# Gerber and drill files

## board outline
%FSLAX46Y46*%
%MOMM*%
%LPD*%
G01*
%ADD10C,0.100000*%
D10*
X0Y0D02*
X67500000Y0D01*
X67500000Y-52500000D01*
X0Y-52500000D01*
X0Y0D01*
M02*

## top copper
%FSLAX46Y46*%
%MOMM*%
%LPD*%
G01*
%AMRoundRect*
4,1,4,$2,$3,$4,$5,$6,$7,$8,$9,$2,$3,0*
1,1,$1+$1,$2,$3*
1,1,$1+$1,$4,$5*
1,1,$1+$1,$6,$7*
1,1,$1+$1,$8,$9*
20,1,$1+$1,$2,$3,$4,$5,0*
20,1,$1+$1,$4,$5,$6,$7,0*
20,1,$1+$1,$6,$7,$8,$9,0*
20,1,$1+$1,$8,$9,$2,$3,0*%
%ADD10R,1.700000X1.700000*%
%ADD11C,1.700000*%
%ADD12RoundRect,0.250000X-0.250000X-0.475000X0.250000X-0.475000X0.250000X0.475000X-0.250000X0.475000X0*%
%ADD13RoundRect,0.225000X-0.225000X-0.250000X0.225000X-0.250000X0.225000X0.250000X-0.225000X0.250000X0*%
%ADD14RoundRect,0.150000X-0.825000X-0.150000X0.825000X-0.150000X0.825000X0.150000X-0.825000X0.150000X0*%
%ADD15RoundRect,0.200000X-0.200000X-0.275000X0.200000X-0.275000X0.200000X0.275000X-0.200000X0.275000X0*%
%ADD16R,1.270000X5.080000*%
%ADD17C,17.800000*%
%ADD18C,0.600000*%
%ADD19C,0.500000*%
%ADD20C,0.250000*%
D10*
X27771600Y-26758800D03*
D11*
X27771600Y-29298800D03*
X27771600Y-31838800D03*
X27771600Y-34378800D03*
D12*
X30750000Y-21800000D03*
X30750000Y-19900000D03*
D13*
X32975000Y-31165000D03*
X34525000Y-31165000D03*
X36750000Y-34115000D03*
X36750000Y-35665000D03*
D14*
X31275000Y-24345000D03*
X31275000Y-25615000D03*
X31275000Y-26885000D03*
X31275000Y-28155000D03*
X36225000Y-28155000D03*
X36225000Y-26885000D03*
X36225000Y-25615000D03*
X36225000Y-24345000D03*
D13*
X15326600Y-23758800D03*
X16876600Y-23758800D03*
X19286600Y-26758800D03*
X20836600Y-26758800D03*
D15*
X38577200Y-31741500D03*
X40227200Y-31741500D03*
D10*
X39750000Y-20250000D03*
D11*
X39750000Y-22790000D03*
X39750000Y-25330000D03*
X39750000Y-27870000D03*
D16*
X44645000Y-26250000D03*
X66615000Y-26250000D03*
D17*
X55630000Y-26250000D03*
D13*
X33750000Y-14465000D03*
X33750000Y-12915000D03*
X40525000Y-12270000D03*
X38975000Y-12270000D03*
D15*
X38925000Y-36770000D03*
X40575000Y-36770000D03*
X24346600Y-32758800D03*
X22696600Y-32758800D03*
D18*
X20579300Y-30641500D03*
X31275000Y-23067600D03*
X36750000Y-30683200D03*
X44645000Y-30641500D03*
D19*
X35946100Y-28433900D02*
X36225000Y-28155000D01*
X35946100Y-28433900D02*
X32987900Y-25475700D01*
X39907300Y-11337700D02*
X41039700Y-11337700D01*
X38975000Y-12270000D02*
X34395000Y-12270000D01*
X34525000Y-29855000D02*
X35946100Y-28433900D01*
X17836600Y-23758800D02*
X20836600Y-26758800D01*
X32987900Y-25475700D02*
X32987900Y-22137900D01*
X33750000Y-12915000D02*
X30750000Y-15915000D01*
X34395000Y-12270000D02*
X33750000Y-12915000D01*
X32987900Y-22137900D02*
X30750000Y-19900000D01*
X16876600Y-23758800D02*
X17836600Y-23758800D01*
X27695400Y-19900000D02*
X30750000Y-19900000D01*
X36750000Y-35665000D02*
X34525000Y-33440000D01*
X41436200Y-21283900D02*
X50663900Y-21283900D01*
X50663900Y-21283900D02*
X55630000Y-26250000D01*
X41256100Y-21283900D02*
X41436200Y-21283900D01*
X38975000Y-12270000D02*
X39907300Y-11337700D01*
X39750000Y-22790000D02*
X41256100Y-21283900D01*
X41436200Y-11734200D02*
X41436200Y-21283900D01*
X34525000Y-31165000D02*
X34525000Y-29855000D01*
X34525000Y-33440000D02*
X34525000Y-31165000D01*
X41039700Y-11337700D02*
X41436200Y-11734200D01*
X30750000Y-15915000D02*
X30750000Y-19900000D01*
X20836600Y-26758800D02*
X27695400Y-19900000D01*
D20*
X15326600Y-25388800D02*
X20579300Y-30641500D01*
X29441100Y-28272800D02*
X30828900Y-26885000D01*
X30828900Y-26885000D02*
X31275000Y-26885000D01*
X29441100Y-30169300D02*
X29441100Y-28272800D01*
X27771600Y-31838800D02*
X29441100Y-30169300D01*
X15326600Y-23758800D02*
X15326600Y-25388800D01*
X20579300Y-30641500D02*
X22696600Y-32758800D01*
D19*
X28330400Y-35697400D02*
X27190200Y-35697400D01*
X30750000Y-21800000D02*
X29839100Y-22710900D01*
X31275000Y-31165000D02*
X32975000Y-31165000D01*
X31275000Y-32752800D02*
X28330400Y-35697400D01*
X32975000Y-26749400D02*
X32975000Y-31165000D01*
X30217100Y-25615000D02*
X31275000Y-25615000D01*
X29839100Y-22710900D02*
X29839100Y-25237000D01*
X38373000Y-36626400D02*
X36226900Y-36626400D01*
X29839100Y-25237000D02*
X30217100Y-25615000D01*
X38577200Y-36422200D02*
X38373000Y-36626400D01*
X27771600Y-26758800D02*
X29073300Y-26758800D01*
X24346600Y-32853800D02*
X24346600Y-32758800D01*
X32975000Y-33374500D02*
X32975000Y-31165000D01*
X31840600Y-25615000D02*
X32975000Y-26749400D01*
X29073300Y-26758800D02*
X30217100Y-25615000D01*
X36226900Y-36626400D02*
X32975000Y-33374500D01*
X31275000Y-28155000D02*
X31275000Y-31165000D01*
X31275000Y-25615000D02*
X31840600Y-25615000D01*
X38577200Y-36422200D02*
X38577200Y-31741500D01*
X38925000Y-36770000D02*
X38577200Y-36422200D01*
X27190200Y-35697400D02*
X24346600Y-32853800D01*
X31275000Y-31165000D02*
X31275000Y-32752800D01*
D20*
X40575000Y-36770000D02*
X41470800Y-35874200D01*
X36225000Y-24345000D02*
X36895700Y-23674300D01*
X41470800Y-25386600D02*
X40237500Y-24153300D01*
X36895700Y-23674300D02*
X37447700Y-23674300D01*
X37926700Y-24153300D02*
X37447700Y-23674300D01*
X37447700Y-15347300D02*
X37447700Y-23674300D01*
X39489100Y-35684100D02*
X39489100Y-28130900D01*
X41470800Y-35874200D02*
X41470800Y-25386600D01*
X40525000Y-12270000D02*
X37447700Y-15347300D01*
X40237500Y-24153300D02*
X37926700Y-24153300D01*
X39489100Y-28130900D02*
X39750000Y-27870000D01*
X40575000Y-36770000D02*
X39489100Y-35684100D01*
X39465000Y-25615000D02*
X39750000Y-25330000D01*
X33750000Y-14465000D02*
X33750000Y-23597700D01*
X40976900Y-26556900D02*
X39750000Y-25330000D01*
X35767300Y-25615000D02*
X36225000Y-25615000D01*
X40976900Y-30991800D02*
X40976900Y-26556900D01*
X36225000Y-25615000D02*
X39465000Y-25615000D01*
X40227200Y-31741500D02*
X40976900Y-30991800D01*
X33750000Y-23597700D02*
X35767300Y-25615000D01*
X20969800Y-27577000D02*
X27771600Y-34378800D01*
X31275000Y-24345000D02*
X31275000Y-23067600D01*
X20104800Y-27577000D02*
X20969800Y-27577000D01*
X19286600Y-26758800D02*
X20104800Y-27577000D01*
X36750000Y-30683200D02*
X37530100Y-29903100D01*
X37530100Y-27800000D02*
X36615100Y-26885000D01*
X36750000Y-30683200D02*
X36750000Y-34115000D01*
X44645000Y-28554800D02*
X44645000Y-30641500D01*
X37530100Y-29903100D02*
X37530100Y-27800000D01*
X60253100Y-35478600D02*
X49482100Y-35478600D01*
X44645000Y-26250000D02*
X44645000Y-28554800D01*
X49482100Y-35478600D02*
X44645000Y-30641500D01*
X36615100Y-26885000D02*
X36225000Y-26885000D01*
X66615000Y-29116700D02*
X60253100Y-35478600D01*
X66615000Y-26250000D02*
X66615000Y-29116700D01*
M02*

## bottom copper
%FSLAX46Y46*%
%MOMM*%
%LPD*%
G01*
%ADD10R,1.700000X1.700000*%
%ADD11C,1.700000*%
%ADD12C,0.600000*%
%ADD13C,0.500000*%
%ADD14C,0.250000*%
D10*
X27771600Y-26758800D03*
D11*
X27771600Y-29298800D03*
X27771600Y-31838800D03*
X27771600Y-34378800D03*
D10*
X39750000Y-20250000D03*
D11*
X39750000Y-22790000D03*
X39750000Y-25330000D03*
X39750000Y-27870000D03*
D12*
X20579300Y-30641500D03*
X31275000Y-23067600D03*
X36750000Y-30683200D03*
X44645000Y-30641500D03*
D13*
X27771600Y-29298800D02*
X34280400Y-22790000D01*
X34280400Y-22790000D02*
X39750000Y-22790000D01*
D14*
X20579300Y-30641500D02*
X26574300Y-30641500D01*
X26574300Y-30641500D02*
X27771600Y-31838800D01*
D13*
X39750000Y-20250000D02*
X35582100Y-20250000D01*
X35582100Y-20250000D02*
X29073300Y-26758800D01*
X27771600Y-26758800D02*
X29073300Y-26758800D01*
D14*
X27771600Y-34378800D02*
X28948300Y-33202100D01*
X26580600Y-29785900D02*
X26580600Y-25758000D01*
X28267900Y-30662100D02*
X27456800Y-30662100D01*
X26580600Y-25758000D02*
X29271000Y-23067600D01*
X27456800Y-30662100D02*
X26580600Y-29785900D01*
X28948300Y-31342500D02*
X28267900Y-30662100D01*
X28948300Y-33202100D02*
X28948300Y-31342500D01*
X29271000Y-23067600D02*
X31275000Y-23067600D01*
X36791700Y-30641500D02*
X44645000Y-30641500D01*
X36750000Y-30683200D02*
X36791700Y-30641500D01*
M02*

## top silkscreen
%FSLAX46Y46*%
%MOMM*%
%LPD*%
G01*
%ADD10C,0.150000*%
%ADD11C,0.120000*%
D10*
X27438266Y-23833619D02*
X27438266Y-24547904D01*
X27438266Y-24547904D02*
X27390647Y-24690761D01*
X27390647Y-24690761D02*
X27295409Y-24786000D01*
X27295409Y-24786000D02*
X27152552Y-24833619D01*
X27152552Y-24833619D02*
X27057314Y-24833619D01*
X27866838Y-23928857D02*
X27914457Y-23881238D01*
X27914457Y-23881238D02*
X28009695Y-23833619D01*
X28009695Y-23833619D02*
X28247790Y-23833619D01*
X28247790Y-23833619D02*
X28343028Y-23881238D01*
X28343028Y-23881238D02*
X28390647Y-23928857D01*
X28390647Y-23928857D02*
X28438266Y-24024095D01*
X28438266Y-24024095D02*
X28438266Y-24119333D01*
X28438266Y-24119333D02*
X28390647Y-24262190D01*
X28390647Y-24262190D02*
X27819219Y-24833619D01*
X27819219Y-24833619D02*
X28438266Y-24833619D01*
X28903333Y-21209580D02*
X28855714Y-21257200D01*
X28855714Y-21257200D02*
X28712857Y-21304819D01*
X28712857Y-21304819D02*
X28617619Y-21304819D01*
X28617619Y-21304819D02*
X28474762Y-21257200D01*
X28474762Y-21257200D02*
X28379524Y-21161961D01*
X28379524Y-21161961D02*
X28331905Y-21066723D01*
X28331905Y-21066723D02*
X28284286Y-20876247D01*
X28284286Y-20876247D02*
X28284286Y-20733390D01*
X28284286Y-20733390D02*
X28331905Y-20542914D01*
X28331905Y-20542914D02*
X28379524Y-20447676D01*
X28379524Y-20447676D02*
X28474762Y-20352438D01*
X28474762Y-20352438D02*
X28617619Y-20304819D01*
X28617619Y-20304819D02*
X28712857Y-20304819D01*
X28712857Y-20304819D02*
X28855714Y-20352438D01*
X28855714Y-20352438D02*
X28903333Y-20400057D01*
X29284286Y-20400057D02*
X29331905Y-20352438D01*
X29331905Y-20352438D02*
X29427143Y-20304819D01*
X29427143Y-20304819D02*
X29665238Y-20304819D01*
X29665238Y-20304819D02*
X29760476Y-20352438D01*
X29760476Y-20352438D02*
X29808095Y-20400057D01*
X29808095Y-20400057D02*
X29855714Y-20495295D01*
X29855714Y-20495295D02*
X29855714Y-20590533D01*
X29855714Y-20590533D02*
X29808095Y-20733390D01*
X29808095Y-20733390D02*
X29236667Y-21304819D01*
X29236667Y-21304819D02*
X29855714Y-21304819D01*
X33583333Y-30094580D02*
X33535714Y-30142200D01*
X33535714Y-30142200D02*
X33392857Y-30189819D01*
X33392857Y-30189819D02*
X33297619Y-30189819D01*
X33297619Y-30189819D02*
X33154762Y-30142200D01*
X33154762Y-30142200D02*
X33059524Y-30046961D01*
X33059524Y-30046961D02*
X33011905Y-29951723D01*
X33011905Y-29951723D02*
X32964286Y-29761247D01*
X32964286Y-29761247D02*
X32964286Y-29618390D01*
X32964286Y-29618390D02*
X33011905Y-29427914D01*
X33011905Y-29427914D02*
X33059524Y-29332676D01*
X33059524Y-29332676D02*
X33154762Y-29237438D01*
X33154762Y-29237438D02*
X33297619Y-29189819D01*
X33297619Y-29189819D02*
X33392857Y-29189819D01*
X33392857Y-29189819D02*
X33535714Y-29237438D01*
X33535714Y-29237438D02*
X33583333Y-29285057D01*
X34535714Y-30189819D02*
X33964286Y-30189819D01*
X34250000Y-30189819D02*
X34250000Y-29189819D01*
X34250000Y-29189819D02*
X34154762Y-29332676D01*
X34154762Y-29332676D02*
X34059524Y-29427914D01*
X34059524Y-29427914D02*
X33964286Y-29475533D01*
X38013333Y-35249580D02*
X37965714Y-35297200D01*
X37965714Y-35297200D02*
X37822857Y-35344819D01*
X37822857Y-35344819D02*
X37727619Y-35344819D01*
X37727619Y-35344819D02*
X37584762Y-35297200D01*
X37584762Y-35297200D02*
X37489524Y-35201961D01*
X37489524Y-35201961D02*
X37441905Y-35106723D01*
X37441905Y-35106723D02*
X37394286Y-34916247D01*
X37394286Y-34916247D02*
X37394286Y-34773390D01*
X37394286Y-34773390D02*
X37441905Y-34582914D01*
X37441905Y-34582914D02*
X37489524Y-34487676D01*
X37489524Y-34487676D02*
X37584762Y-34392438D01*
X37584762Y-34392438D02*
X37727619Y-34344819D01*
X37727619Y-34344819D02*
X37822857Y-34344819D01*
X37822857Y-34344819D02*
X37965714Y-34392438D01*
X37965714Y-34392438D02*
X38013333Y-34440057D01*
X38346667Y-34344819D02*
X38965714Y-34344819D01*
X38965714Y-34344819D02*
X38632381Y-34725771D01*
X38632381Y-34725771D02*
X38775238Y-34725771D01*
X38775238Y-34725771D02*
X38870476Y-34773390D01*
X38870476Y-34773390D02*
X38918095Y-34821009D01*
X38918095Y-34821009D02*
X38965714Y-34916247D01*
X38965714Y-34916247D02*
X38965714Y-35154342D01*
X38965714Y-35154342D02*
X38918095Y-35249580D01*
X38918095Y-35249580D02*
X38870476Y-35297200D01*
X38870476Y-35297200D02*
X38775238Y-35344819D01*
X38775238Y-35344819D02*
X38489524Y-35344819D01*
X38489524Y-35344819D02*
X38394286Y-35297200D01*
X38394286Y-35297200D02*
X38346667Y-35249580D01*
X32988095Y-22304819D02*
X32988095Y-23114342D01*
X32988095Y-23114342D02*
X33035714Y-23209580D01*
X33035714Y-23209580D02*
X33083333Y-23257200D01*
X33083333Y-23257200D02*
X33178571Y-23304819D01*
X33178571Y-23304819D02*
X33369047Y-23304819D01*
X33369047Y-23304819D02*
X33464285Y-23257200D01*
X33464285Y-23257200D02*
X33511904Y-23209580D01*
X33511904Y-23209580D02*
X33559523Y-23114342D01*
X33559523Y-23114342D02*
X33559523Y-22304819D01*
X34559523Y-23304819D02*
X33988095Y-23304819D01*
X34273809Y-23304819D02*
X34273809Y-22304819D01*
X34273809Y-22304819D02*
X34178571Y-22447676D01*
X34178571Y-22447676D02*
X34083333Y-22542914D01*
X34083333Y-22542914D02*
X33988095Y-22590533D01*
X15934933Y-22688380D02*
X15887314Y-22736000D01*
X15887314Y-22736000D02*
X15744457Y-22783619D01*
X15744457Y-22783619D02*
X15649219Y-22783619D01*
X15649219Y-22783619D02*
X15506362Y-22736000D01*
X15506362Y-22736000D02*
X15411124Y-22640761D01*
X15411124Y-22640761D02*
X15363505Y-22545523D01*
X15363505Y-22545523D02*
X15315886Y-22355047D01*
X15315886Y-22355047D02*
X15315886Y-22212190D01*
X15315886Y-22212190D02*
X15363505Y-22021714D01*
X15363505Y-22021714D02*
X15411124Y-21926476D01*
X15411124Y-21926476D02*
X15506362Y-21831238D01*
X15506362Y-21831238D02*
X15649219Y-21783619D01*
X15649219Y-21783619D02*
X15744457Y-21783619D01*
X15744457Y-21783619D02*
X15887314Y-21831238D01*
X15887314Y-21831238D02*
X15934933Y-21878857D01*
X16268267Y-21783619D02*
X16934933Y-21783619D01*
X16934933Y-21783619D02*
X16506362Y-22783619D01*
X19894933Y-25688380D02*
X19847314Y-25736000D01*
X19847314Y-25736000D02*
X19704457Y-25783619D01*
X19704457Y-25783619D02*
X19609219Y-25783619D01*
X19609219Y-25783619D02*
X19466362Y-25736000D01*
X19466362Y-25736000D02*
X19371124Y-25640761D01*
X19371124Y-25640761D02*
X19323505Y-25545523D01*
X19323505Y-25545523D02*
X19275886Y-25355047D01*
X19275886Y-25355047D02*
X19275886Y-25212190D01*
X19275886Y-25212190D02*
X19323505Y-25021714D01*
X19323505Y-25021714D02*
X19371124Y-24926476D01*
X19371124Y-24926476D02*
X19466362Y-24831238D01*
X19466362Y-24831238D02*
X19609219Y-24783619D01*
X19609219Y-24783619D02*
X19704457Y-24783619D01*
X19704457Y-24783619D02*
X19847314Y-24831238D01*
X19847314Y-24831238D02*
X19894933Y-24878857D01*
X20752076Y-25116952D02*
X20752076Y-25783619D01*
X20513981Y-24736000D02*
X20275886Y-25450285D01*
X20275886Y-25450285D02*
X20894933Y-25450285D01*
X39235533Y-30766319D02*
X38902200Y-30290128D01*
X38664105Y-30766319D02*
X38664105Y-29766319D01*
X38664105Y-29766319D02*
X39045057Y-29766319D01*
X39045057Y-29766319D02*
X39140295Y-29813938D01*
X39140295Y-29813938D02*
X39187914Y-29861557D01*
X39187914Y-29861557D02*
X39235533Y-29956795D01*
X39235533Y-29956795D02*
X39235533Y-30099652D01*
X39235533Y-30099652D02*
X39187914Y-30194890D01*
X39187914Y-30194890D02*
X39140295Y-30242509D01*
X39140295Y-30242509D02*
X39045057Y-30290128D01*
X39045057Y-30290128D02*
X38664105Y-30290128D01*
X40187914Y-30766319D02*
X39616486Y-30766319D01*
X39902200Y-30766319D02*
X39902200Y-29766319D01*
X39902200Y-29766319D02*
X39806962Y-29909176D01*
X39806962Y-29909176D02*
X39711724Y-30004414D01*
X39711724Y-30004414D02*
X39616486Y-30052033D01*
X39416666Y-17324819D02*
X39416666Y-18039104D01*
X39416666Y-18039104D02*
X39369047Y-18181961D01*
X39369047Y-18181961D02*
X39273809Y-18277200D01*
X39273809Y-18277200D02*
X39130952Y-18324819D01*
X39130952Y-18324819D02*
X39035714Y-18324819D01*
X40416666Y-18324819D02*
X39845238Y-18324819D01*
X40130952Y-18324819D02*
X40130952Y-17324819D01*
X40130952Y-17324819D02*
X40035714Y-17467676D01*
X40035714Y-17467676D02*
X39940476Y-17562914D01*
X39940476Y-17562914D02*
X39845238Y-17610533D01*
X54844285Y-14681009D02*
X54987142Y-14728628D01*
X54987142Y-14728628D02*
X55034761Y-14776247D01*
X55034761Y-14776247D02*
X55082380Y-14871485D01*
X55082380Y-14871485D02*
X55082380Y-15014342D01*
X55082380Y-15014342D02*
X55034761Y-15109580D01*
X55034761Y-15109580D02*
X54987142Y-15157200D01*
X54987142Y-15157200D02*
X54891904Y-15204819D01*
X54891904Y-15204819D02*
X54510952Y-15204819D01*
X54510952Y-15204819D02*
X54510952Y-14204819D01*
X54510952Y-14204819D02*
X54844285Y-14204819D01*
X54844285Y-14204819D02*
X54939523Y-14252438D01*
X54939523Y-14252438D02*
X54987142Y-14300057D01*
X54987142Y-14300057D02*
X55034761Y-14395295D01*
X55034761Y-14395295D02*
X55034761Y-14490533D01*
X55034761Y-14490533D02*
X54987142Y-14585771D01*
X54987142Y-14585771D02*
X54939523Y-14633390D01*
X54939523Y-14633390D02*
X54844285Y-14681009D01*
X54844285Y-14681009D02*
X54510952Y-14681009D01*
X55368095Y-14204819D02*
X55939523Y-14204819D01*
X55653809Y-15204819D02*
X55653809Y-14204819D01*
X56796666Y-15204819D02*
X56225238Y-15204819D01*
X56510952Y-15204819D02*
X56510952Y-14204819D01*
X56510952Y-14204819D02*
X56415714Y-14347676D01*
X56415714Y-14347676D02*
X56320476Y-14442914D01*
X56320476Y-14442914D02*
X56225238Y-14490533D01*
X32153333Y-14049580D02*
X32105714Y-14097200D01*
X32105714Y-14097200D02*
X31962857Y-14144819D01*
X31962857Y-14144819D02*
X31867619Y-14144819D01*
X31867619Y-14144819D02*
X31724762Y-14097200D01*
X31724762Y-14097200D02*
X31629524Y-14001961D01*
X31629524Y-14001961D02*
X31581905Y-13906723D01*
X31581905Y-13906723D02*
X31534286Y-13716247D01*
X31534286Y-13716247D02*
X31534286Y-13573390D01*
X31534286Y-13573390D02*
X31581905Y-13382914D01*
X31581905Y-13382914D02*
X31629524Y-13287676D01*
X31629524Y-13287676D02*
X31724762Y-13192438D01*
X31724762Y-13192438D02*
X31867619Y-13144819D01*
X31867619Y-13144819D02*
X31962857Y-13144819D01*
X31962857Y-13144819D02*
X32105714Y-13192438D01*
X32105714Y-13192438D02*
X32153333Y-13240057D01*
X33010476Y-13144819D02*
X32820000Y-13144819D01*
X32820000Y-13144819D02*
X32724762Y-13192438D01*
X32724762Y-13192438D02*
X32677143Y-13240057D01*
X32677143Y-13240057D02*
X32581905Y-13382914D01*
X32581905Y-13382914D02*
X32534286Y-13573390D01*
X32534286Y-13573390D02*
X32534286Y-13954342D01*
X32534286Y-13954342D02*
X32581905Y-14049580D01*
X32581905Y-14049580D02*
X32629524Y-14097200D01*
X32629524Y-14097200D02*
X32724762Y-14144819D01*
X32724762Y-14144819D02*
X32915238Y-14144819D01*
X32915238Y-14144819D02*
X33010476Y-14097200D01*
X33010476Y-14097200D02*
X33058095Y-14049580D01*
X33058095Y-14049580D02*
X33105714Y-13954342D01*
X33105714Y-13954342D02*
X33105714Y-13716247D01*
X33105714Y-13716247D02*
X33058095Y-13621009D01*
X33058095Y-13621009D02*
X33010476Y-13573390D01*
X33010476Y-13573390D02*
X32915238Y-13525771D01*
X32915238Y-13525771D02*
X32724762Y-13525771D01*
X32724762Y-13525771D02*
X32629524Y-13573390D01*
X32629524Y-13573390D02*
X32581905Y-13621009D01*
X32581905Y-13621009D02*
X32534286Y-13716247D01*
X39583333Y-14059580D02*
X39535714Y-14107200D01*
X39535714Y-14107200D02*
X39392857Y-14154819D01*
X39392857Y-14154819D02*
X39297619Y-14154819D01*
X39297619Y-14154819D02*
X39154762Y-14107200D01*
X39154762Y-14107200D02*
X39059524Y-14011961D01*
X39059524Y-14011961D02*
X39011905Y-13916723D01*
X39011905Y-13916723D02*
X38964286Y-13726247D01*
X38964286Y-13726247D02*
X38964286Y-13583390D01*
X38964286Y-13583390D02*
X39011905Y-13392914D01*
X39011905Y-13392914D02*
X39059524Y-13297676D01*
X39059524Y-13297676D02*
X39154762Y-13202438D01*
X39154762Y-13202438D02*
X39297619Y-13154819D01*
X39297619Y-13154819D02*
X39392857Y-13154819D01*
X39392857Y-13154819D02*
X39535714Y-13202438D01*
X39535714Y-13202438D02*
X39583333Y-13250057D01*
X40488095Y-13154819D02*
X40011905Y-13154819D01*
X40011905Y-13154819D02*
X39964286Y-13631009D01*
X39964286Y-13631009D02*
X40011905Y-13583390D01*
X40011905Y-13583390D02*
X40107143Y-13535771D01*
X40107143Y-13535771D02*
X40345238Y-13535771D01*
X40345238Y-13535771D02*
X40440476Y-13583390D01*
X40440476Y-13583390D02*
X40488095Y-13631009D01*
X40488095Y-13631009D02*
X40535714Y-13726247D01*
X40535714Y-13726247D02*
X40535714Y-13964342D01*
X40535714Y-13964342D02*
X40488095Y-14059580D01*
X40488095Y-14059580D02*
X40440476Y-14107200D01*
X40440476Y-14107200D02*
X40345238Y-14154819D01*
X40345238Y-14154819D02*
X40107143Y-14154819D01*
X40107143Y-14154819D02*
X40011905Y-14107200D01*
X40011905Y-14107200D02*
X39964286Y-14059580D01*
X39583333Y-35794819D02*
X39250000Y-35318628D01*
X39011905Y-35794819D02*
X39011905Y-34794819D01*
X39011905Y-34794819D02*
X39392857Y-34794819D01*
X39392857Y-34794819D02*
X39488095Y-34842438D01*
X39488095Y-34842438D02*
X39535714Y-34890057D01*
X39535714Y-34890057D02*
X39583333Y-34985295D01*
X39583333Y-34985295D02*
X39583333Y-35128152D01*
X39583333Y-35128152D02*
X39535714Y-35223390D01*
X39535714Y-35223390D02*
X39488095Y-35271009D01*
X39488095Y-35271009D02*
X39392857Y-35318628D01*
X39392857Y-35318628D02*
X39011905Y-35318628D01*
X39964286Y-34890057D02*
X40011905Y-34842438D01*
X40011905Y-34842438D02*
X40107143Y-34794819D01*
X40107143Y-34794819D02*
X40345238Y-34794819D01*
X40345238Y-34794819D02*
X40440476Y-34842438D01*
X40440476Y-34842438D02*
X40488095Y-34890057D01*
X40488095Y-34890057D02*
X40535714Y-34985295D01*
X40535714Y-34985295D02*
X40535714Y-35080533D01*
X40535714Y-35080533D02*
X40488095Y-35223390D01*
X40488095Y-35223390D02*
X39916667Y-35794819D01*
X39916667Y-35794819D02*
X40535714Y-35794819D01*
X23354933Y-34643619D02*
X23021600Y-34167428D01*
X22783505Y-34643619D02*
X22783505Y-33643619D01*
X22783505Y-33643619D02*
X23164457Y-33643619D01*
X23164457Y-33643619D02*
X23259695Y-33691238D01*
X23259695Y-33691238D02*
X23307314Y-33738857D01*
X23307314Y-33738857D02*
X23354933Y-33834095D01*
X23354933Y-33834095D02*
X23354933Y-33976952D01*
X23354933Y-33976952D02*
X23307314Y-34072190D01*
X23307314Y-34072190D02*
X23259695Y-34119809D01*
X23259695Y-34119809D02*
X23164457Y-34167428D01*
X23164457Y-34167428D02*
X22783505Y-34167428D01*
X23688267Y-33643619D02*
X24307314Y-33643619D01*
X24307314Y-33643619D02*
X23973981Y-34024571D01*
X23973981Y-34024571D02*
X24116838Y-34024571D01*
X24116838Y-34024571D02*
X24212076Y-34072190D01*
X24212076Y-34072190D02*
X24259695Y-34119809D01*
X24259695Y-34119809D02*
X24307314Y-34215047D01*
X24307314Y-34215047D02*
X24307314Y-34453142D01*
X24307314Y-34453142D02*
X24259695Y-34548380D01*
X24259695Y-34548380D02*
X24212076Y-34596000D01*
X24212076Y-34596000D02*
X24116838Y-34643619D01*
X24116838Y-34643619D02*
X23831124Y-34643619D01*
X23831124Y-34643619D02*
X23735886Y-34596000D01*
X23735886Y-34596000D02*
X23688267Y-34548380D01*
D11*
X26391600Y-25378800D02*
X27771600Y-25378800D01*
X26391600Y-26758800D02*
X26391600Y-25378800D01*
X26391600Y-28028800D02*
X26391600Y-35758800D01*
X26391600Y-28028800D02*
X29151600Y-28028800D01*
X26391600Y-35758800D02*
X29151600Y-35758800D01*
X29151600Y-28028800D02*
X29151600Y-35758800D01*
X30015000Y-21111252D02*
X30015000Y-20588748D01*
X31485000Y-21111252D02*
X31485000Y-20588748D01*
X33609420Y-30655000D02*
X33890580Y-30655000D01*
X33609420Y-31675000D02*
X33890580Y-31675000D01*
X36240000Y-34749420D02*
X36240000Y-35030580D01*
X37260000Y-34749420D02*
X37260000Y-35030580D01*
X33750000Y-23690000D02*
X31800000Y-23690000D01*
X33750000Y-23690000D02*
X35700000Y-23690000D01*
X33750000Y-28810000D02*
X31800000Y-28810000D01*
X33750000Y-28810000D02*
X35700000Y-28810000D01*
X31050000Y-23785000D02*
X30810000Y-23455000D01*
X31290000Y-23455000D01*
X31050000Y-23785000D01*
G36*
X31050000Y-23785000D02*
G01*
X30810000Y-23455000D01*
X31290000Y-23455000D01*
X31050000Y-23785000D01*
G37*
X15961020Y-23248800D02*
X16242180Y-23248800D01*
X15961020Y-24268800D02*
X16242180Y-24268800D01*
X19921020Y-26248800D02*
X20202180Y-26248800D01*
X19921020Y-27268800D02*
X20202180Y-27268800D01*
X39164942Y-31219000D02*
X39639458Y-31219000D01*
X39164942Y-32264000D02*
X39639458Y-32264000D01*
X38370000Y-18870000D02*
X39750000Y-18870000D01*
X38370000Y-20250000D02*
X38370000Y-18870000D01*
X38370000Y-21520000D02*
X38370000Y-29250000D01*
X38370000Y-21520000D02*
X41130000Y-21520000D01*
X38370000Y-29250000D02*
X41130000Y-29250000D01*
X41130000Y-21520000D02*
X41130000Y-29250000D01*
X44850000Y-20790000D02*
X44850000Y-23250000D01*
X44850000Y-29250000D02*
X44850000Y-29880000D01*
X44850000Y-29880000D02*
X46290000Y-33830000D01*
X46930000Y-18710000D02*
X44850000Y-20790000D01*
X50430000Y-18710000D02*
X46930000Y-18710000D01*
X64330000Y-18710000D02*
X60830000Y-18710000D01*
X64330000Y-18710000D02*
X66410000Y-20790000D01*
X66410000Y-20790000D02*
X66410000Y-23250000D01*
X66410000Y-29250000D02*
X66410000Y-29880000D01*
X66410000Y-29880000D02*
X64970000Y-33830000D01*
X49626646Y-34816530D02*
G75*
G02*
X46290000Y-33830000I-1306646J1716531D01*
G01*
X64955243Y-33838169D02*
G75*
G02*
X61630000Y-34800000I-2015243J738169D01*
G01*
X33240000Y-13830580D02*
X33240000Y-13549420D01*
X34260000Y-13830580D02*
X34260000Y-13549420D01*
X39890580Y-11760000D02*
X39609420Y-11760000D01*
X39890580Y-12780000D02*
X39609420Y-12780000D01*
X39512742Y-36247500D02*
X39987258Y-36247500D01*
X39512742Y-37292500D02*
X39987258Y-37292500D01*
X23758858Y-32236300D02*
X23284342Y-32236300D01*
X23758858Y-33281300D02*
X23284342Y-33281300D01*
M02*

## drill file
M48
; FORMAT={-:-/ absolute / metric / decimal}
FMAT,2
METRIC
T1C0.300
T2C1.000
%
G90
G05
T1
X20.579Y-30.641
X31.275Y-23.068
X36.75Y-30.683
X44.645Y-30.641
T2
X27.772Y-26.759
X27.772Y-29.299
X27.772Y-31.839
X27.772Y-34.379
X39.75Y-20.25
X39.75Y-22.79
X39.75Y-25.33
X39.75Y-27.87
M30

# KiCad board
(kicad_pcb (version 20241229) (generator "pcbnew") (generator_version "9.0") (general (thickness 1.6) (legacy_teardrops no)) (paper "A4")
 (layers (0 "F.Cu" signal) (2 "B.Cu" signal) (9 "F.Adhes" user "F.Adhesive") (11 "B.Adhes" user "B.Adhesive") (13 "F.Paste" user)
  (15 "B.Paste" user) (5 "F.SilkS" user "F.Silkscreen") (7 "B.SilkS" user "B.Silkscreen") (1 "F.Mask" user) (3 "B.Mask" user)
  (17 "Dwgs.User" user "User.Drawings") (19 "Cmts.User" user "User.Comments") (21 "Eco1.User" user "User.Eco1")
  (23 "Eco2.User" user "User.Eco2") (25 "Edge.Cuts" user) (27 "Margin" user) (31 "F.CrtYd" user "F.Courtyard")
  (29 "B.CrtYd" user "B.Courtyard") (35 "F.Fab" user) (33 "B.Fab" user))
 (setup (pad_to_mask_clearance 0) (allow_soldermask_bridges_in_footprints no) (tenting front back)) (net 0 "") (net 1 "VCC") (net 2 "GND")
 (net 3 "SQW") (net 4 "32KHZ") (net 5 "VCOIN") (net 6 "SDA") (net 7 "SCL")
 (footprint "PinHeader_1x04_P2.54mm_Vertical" (layer "F.Cu") (at 27.7716 26.7588)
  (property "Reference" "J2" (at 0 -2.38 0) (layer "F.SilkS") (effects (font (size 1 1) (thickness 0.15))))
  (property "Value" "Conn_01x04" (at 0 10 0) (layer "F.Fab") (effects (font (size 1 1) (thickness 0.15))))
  (fp_line (start -1.38 -1.38) (end 0 -1.38) (stroke (width 0.12) (type solid)) (layer "F.SilkS"))
  (fp_line (start -1.38 0) (end -1.38 -1.38) (stroke (width 0.12) (type solid)) (layer "F.SilkS"))
  (fp_line (start -1.38 1.27) (end -1.38 9) (stroke (width 0.12) (type solid)) (layer "F.SilkS"))
  (fp_line (start -1.38 1.27) (end 1.38 1.27) (stroke (width 0.12) (type solid)) (layer "F.SilkS"))
  (fp_line (start -1.38 9) (end 1.38 9) (stroke (width 0.12) (type solid)) (layer "F.SilkS"))
  (fp_line (start 1.38 1.27) (end 1.38 9) (stroke (width 0.12) (type solid)) (layer "F.SilkS"))
  (pad "1" thru_hole rect (at 0 0) (size 1.7 1.7) (drill 1) (layers "*.Cu" "*.Mask") (remove_unused_layers no) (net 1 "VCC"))
  (pad "2" thru_hole circle (at 0 2.54) (size 1.7 1.7) (drill 1) (layers "*.Cu" "*.Mask") (remove_unused_layers no) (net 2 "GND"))
  (pad "3" thru_hole circle (at 0 5.08) (size 1.7 1.7) (drill 1) (layers "*.Cu" "*.Mask") (remove_unused_layers no) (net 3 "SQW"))
  (pad "4" thru_hole circle (at 0 7.62) (size 1.7 1.7) (drill 1) (layers "*.Cu" "*.Mask") (remove_unused_layers no) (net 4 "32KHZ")))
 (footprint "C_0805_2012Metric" (layer "F.Cu") (at 30.75 20.85 90)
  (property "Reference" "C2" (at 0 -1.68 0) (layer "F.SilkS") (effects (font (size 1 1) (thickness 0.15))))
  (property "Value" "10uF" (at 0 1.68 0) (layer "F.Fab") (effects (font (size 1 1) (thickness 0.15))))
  (fp_line (start -0.261252 -0.735) (end 0.261252 -0.735) (stroke (width 0.12) (type solid)) (layer "F.SilkS"))
  (fp_line (start -0.261252 0.735) (end 0.261252 0.735) (stroke (width 0.12) (type solid)) (layer "F.SilkS"))
  (pad "1" smd roundrect (at -0.95 0) (size 1 1.45) (layers "F.Cu" "F.Mask" "F.Paste") (roundrect_rratio 0.25) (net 1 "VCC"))
  (pad "2" smd roundrect (at 0.95 0) (size 1 1.45) (layers "F.Cu" "F.Mask" "F.Paste") (roundrect_rratio 0.25) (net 2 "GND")))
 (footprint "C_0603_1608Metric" (layer "F.Cu") (at 33.75 31.165)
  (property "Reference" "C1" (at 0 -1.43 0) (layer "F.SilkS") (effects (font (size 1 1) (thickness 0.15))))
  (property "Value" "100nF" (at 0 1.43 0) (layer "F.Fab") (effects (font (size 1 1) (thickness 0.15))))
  (fp_line (start -0.14058 -0.51) (end 0.14058 -0.51) (stroke (width 0.12) (type solid)) (layer "F.SilkS"))
  (fp_line (start -0.14058 0.51) (end 0.14058 0.51) (stroke (width 0.12) (type solid)) (layer "F.SilkS"))
  (pad "1" smd roundrect (at -0.775 0) (size 0.9 0.95) (layers "F.Cu" "F.Mask" "F.Paste") (roundrect_rratio 0.25) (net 1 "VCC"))
  (pad "2" smd roundrect (at 0.775 0) (size 0.9 0.95) (layers "F.Cu" "F.Mask" "F.Paste") (roundrect_rratio 0.25) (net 2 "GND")))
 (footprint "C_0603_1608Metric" (layer "F.Cu") (at 36.75 34.89 -90)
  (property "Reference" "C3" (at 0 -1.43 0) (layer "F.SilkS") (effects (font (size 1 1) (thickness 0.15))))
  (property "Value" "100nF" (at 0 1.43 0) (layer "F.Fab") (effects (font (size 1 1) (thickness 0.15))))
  (fp_line (start -0.14058 0.51) (end 0.14058 0.51) (stroke (width 0.12) (type solid)) (layer "F.SilkS"))
  (fp_line (start -0.14058 -0.51) (end 0.14058 -0.51) (stroke (width 0.12) (type solid)) (layer "F.SilkS"))
  (pad "1" smd roundrect (at -0.775 0) (size 0.9 0.95) (layers "F.Cu" "F.Mask" "F.Paste") (roundrect_rratio 0.25) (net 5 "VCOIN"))
  (pad "2" smd roundrect (at 0.775 0) (size 0.9 0.95) (layers "F.Cu" "F.Mask" "F.Paste") (roundrect_rratio 0.25) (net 2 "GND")))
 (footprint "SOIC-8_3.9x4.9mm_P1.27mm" (layer "F.Cu") (at 33.75 26.25)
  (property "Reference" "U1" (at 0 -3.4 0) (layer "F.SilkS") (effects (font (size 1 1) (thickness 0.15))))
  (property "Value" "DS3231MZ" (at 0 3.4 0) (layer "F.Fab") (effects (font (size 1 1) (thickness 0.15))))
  (fp_line (start 0 -2.56) (end -1.95 -2.56) (stroke (width 0.12) (type solid)) (layer "F.SilkS"))
  (fp_line (start 0 -2.56) (end 1.95 -2.56) (stroke (width 0.12) (type solid)) (layer "F.SilkS"))
  (fp_line (start 0 2.56) (end -1.95 2.56) (stroke (width 0.12) (type solid)) (layer "F.SilkS"))
  (fp_line (start 0 2.56) (end 1.95 2.56) (stroke (width 0.12) (type solid)) (layer "F.SilkS"))
  (fp_poly (pts (xy -2.7 -2.465) (xy -2.94 -2.795) (xy -2.46 -2.795)) (stroke (width 0.12) (type solid)) (fill yes) (layer "F.SilkS"))
  (pad "1" smd roundrect (at -2.475 -1.905) (size 1.95 0.6) (layers "F.Cu" "F.Mask" "F.Paste") (roundrect_rratio 0.25) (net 4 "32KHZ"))
  (pad "2" smd roundrect (at -2.475 -0.635) (size 1.95 0.6) (layers "F.Cu" "F.Mask" "F.Paste") (roundrect_rratio 0.25) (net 1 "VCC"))
  (pad "3" smd roundrect (at -2.475 0.635) (size 1.95 0.6) (layers "F.Cu" "F.Mask" "F.Paste") (roundrect_rratio 0.25) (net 3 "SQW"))
  (pad "4" smd roundrect (at -2.475 1.905) (size 1.95 0.6) (layers "F.Cu" "F.Mask" "F.Paste") (roundrect_rratio 0.25) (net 1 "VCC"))
  (pad "5" smd roundrect (at 2.475 1.905) (size 1.95 0.6) (layers "F.Cu" "F.Mask" "F.Paste") (roundrect_rratio 0.25) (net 2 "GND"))
  (pad "6" smd roundrect (at 2.475 0.635) (size 1.95 0.6) (layers "F.Cu" "F.Mask" "F.Paste") (roundrect_rratio 0.25) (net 5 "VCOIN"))
  (pad "7" smd roundrect (at 2.475 -0.635) (size 1.95 0.6) (layers "F.Cu" "F.Mask" "F.Paste") (roundrect_rratio 0.25) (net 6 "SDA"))
  (pad "8" smd roundrect (at 2.475 -1.905) (size 1.95 0.6) (layers "F.Cu" "F.Mask" "F.Paste") (roundrect_rratio 0.25) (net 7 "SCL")))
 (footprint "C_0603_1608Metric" (layer "F.Cu") (at 16.1016 23.7588)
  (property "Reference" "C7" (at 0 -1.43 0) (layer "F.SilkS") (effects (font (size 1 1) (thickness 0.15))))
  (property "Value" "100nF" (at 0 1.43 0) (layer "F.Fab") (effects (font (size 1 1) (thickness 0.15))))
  (fp_line (start -0.14058 -0.51) (end 0.14058 -0.51) (stroke (width 0.12) (type solid)) (layer "F.SilkS"))
  (fp_line (start -0.14058 0.51) (end 0.14058 0.51) (stroke (width 0.12) (type solid)) (layer "F.SilkS"))
  (pad "1" smd roundrect (at -0.775 0) (size 0.9 0.95) (layers "F.Cu" "F.Mask" "F.Paste") (roundrect_rratio 0.25) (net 3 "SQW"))
  (pad "2" smd roundrect (at 0.775 0) (size 0.9 0.95) (layers "F.Cu" "F.Mask" "F.Paste") (roundrect_rratio 0.25) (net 2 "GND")))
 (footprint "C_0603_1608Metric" (layer "F.Cu") (at 20.0616 26.7588)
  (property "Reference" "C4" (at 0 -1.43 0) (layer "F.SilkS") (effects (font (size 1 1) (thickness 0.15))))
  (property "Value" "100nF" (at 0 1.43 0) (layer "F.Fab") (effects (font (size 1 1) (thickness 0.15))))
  (fp_line (start -0.14058 -0.51) (end 0.14058 -0.51) (stroke (width 0.12) (type solid)) (layer "F.SilkS"))
  (fp_line (start -0.14058 0.51) (end 0.14058 0.51) (stroke (width 0.12) (type solid)) (layer "F.SilkS"))
  (pad "1" smd roundrect (at -0.775 0) (size 0.9 0.95) (layers "F.Cu" "F.Mask" "F.Paste") (roundrect_rratio 0.25) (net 4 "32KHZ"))
  (pad "2" smd roundrect (at 0.775 0) (size 0.9 0.95) (layers "F.Cu" "F.Mask" "F.Paste") (roundrect_rratio 0.25) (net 2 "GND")))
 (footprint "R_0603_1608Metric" (layer "F.Cu") (at 39.4022 31.7415)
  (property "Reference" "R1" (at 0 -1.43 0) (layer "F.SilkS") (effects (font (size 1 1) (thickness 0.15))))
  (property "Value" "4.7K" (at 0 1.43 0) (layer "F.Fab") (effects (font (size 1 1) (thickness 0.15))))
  (fp_line (start -0.237258 -0.5225) (end 0.237258 -0.5225) (stroke (width 0.12) (type solid)) (layer "F.SilkS"))
  (fp_line (start -0.237258 0.5225) (end 0.237258 0.5225) (stroke (width 0.12) (type solid)) (layer "F.SilkS"))
  (pad "1" smd roundrect (at -0.825 0) (size 0.8 0.95) (layers "F.Cu" "F.Mask" "F.Paste") (roundrect_rratio 0.25) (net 1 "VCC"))
  (pad "2" smd roundrect (at 0.825 0) (size 0.8 0.95) (layers "F.Cu" "F.Mask" "F.Paste") (roundrect_rratio 0.25) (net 6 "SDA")))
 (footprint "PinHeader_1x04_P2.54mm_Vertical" (layer "F.Cu") (at 39.75 20.25)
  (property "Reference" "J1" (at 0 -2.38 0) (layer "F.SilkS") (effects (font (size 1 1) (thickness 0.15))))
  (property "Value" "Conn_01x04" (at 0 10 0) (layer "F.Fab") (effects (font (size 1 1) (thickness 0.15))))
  (fp_line (start -1.38 -1.38) (end 0 -1.38) (stroke (width 0.12) (type solid)) (layer "F.SilkS"))
  (fp_line (start -1.38 0) (end -1.38 -1.38) (stroke (width 0.12) (type solid)) (layer "F.SilkS"))
  (fp_line (start -1.38 1.27) (end -1.38 9) (stroke (width 0.12) (type solid)) (layer "F.SilkS"))
  (fp_line (start -1.38 1.27) (end 1.38 1.27) (stroke (width 0.12) (type solid)) (layer "F.SilkS"))
  (fp_line (start -1.38 9) (end 1.38 9) (stroke (width 0.12) (type solid)) (layer "F.SilkS"))
  (fp_line (start 1.38 1.27) (end 1.38 9) (stroke (width 0.12) (type solid)) (layer "F.SilkS"))
  (pad "1" thru_hole rect (at 0 0) (size 1.7 1.7) (drill 1) (layers "*.Cu" "*.Mask") (remove_unused_layers no) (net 1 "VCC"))
  (pad "2" thru_hole circle (at 0 2.54) (size 1.7 1.7) (drill 1) (layers "*.Cu" "*.Mask") (remove_unused_layers no) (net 2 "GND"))
  (pad "3" thru_hole circle (at 0 5.08) (size 1.7 1.7) (drill 1) (layers "*.Cu" "*.Mask") (remove_unused_layers no) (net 6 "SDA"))
  (pad "4" thru_hole circle (at 0 7.62) (size 1.7 1.7) (drill 1) (layers "*.Cu" "*.Mask") (remove_unused_layers no) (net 7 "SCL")))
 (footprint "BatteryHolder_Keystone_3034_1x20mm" (layer "F.Cu") (at 55.63 26.25)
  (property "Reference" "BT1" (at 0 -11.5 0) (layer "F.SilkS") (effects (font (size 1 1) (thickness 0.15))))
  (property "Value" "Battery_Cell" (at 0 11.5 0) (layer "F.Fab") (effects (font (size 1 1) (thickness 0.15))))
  (fp_line (start -10.78 -5.46) (end -10.78 -3) (stroke (width 0.12) (type solid)) (layer "F.SilkS"))
  (fp_line (start -10.78 3) (end -10.78 3.63) (stroke (width 0.12) (type solid)) (layer "F.SilkS"))
  (fp_line (start -10.78 3.63) (end -9.34 7.58) (stroke (width 0.12) (type solid)) (layer "F.SilkS"))
  (fp_line (start -8.7 -7.54) (end -10.78 -5.46) (stroke (width 0.12) (type solid)) (layer "F.SilkS"))
  (fp_line (start -5.2 -7.54) (end -8.7 -7.54) (stroke (width 0.12) (type solid)) (layer "F.SilkS"))
  (fp_line (start 8.7 -7.54) (end 5.2 -7.54) (stroke (width 0.12) (type solid)) (layer "F.SilkS"))
  (fp_line (start 8.7 -7.54) (end 10.78 -5.46) (stroke (width 0.12) (type solid)) (layer "F.SilkS"))
  (fp_line (start 10.78 -5.46) (end 10.78 -3) (stroke (width 0.12) (type solid)) (layer "F.SilkS"))
  (fp_line (start 10.78 3) (end 10.78 3.63) (stroke (width 0.12) (type solid)) (layer "F.SilkS"))
  (fp_line (start 10.78 3.63) (end 9.34 7.58) (stroke (width 0.12) (type solid)) (layer "F.SilkS"))
  (fp_arc (start -6.003354 8.56653) (mid -7.921654 8.918738) (end -9.34 7.58) (stroke (width 0.12) (type solid)) (layer "F.SilkS"))
  (fp_arc (start 9.325243 7.588169) (mid 7.90634 8.911668) (end 6 8.55) (stroke (width 0.12) (type solid)) (layer "F.SilkS"))
  (pad "1" smd rect (at -10.985 0) (size 1.27 5.08) (layers "F.Cu" "F.Mask" "F.Paste") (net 5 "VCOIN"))
  (pad "1" smd rect (at 10.985 0) (size 1.27 5.08) (layers "F.Cu" "F.Mask" "F.Paste") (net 5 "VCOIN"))
  (pad "2" smd circle (at 0 0) (size 17.8 17.8) (layers "F.Cu" "F.Mask") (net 2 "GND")))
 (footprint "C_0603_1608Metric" (layer "F.Cu") (at 33.75 13.69 90)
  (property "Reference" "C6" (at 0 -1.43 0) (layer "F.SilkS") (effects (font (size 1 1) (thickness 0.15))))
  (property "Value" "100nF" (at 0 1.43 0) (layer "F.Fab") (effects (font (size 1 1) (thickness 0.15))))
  (fp_line (start -0.14058 -0.51) (end 0.14058 -0.51) (stroke (width 0.12) (type solid)) (layer "F.SilkS"))
  (fp_line (start -0.14058 0.51) (end 0.14058 0.51) (stroke (width 0.12) (type solid)) (layer "F.SilkS"))
  (pad "1" smd roundrect (at -0.775 0) (size 0.9 0.95) (layers "F.Cu" "F.Mask" "F.Paste") (roundrect_rratio 0.25) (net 6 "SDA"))
  (pad "2" smd roundrect (at 0.775 0) (size 0.9 0.95) (layers "F.Cu" "F.Mask" "F.Paste") (roundrect_rratio 0.25) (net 2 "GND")))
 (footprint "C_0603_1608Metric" (layer "F.Cu") (at 39.75 12.27 180)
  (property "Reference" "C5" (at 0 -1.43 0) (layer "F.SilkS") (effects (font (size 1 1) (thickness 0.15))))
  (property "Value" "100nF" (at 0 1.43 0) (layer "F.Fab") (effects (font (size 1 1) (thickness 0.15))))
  (fp_line (start -0.14058 0.51) (end 0.14058 0.51) (stroke (width 0.12) (type solid)) (layer "F.SilkS"))
  (fp_line (start -0.14058 -0.51) (end 0.14058 -0.51) (stroke (width 0.12) (type solid)) (layer "F.SilkS"))
  (pad "1" smd roundrect (at -0.775 0) (size 0.9 0.95) (layers "F.Cu" "F.Mask" "F.Paste") (roundrect_rratio 0.25) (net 7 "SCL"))
  (pad "2" smd roundrect (at 0.775 0) (size 0.9 0.95) (layers "F.Cu" "F.Mask" "F.Paste") (roundrect_rratio 0.25) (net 2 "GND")))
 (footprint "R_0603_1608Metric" (layer "F.Cu") (at 39.75 36.77)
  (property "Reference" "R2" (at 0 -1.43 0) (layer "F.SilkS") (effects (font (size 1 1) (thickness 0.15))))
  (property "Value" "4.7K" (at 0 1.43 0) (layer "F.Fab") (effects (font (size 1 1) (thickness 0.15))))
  (fp_line (start -0.237258 -0.5225) (end 0.237258 -0.5225) (stroke (width 0.12) (type solid)) (layer "F.SilkS"))
  (fp_line (start -0.237258 0.5225) (end 0.237258 0.5225) (stroke (width 0.12) (type solid)) (layer "F.SilkS"))
  (pad "1" smd roundrect (at -0.825 0) (size 0.8 0.95) (layers "F.Cu" "F.Mask" "F.Paste") (roundrect_rratio 0.25) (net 1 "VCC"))
  (pad "2" smd roundrect (at 0.825 0) (size 0.8 0.95) (layers "F.Cu" "F.Mask" "F.Paste") (roundrect_rratio 0.25) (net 7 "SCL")))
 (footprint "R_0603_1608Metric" (layer "F.Cu") (at 23.5216 32.7588 180)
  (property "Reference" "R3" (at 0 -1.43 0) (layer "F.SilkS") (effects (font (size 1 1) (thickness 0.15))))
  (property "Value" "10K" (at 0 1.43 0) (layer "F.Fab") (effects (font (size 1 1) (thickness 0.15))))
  (fp_line (start -0.237258 0.5225) (end 0.237258 0.5225) (stroke (width 0.12) (type solid)) (layer "F.SilkS"))
  (fp_line (start -0.237258 -0.5225) (end 0.237258 -0.5225) (stroke (width 0.12) (type solid)) (layer "F.SilkS"))
  (pad "1" smd roundrect (at -0.825 0) (size 0.8 0.95) (layers "F.Cu" "F.Mask" "F.Paste") (roundrect_rratio 0.25) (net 1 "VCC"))
  (pad "2" smd roundrect (at 0.825 0) (size 0.8 0.95) (layers "F.Cu" "F.Mask" "F.Paste") (roundrect_rratio 0.25) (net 3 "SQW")))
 (gr_rect (start 0 0) (end 67.5 52.5) (stroke (width 0.1) (type solid)) (fill no) (layer "Edge.Cuts"))
 (segment (start 35.9461 28.4339) (end 36.225 28.155) (width 0.5) (layer "F.Cu") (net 2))
 (segment (start 35.9461 28.4339) (end 32.9879 25.4757) (width 0.5) (layer "F.Cu") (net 2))
 (segment (start 39.9073 11.3377) (end 41.0397 11.3377) (width 0.5) (layer "F.Cu") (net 2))
 (segment (start 38.975 12.27) (end 34.395 12.27) (width 0.5) (layer "F.Cu") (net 2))
 (segment (start 34.525 29.855) (end 35.9461 28.4339) (width 0.5) (layer "F.Cu") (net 2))
 (segment (start 17.8366 23.7588) (end 20.8366 26.7588) (width 0.5) (layer "F.Cu") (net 2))
 (segment (start 32.9879 25.4757) (end 32.9879 22.1379) (width 0.5) (layer "F.Cu") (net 2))
 (segment (start 33.75 12.915) (end 30.75 15.915) (width 0.5) (layer "F.Cu") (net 2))
 (segment (start 34.395 12.27) (end 33.75 12.915) (width 0.5) (layer "F.Cu") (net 2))
 (segment (start 32.9879 22.1379) (end 30.75 19.9) (width 0.5) (layer "F.Cu") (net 2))
 (segment (start 16.8766 23.7588) (end 17.8366 23.7588) (width 0.5) (layer "F.Cu") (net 2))
 (segment (start 27.6954 19.9) (end 30.75 19.9) (width 0.5) (layer "F.Cu") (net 2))
 (segment (start 36.75 35.665) (end 34.525 33.44) (width 0.5) (layer "F.Cu") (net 2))
 (segment (start 41.4362 21.2839) (end 50.6639 21.2839) (width 0.5) (layer "F.Cu") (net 2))
 (segment (start 50.6639 21.2839) (end 55.63 26.25) (width 0.5) (layer "F.Cu") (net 2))
 (segment (start 41.2561 21.2839) (end 41.4362 21.2839) (width 0.5) (layer "F.Cu") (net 2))
 (segment (start 38.975 12.27) (end 39.9073 11.3377) (width 0.5) (layer "F.Cu") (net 2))
 (segment (start 39.75 22.79) (end 41.2561 21.2839) (width 0.5) (layer "F.Cu") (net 2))
 (segment (start 41.4362 11.7342) (end 41.4362 21.2839) (width 0.5) (layer "F.Cu") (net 2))
 (segment (start 34.525 31.165) (end 34.525 29.855) (width 0.5) (layer "F.Cu") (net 2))
 (segment (start 34.525 33.44) (end 34.525 31.165) (width 0.5) (layer "F.Cu") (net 2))
 (segment (start 41.0397 11.3377) (end 41.4362 11.7342) (width 0.5) (layer "F.Cu") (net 2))
 (segment (start 30.75 15.915) (end 30.75 19.9) (width 0.5) (layer "F.Cu") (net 2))
 (segment (start 20.8366 26.7588) (end 27.6954 19.9) (width 0.5) (layer "F.Cu") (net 2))
 (segment (start 27.7716 29.2988) (end 34.2804 22.79) (width 0.5) (layer "B.Cu") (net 2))
 (segment (start 34.2804 22.79) (end 39.75 22.79) (width 0.5) (layer "B.Cu") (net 2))
 (segment (start 15.3266 25.3888) (end 20.5793 30.6415) (width 0.25) (layer "F.Cu") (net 3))
 (segment (start 29.4411 28.2728) (end 30.8289 26.885) (width 0.25) (layer "F.Cu") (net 3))
 (segment (start 30.8289 26.885) (end 31.275 26.885) (width 0.25) (layer "F.Cu") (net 3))
 (segment (start 29.4411 30.1693) (end 29.4411 28.2728) (width 0.25) (layer "F.Cu") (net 3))
 (segment (start 27.7716 31.8388) (end 29.4411 30.1693) (width 0.25) (layer "F.Cu") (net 3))
 (segment (start 15.3266 23.7588) (end 15.3266 25.3888) (width 0.25) (layer "F.Cu") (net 3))
 (segment (start 20.5793 30.6415) (end 22.6966 32.7588) (width 0.25) (layer "F.Cu") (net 3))
 (via (at 20.5793 30.6415) (size 0.6) (drill 0.3) (layers "F.Cu" "B.Cu") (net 3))
 (segment (start 20.5793 30.6415) (end 26.5743 30.6415) (width 0.25) (layer "B.Cu") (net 3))
 (segment (start 26.5743 30.6415) (end 27.7716 31.8388) (width 0.25) (layer "B.Cu") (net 3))
 (segment (start 28.3304 35.6974) (end 27.1902 35.6974) (width 0.5) (layer "F.Cu") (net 1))
 (segment (start 30.75 21.8) (end 29.8391 22.7109) (width 0.5) (layer "F.Cu") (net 1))
 (segment (start 31.275 31.165) (end 32.975 31.165) (width 0.5) (layer "F.Cu") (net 1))
 (segment (start 31.275 32.7528) (end 28.3304 35.6974) (width 0.5) (layer "F.Cu") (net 1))
 (segment (start 32.975 26.7494) (end 32.975 31.165) (width 0.5) (layer "F.Cu") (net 1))
 (segment (start 30.2171 25.615) (end 31.275 25.615) (width 0.5) (layer "F.Cu") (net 1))
 (segment (start 29.8391 22.7109) (end 29.8391 25.237) (width 0.5) (layer "F.Cu") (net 1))
 (segment (start 38.373 36.6264) (end 36.2269 36.6264) (width 0.5) (layer "F.Cu") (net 1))
 (segment (start 29.8391 25.237) (end 30.2171 25.615) (width 0.5) (layer "F.Cu") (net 1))
 (segment (start 38.5772 36.4222) (end 38.373 36.6264) (width 0.5) (layer "F.Cu") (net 1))
 (segment (start 27.7716 26.7588) (end 29.0733 26.7588) (width 0.5) (layer "F.Cu") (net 1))
 (segment (start 24.3466 32.8538) (end 24.3466 32.7588) (width 0.5) (layer "F.Cu") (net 1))
 (segment (start 32.975 33.3745) (end 32.975 31.165) (width 0.5) (layer "F.Cu") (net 1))
 (segment (start 31.8406 25.615) (end 32.975 26.7494) (width 0.5) (layer "F.Cu") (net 1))
 (segment (start 29.0733 26.7588) (end 30.2171 25.615) (width 0.5) (layer "F.Cu") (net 1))
 (segment (start 36.2269 36.6264) (end 32.975 33.3745) (width 0.5) (layer "F.Cu") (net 1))
 (segment (start 31.275 28.155) (end 31.275 31.165) (width 0.5) (layer "F.Cu") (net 1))
 (segment (start 31.275 25.615) (end 31.8406 25.615) (width 0.5) (layer "F.Cu") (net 1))
 (segment (start 38.5772 36.4222) (end 38.5772 31.7415) (width 0.5) (layer "F.Cu") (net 1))
 (segment (start 38.925 36.77) (end 38.5772 36.4222) (width 0.5) (layer "F.Cu") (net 1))
 (segment (start 27.1902 35.6974) (end 24.3466 32.8538) (width 0.5) (layer "F.Cu") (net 1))
 (segment (start 31.275 31.165) (end 31.275 32.7528) (width 0.5) (layer "F.Cu") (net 1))
 (segment (start 39.75 20.25) (end 35.5821 20.25) (width 0.5) (layer "B.Cu") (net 1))
 (segment (start 35.5821 20.25) (end 29.0733 26.7588) (width 0.5) (layer "B.Cu") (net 1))
 (segment (start 27.7716 26.7588) (end 29.0733 26.7588) (width 0.5) (layer "B.Cu") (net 1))
 (segment (start 40.575 36.77) (end 41.4708 35.8742) (width 0.25) (layer "F.Cu") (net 7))
 (segment (start 36.225 24.345) (end 36.8957 23.6743) (width 0.25) (layer "F.Cu") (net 7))
 (segment (start 41.4708 25.3866) (end 40.2375 24.1533) (width 0.25) (layer "F.Cu") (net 7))
 (segment (start 36.8957 23.6743) (end 37.4477 23.6743) (width 0.25) (layer "F.Cu") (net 7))
 (segment (start 37.9267 24.1533) (end 37.4477 23.6743) (width 0.25) (layer "F.Cu") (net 7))
 (segment (start 37.4477 15.3473) (end 37.4477 23.6743) (width 0.25) (layer "F.Cu") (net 7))
 (segment (start 39.4891 35.6841) (end 39.4891 28.1309) (width 0.25) (layer "F.Cu") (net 7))
 (segment (start 41.4708 35.8742) (end 41.4708 25.3866) (width 0.25) (layer "F.Cu") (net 7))
 (segment (start 40.525 12.27) (end 37.4477 15.3473) (width 0.25) (layer "F.Cu") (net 7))
 (segment (start 40.2375 24.1533) (end 37.9267 24.1533) (width 0.25) (layer "F.Cu") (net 7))
 (segment (start 39.4891 28.1309) (end 39.75 27.87) (width 0.25) (layer "F.Cu") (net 7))
 (segment (start 40.575 36.77) (end 39.4891 35.6841) (width 0.25) (layer "F.Cu") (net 7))
 (segment (start 39.465 25.615) (end 39.75 25.33) (width 0.25) (layer "F.Cu") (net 6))
 (segment (start 33.75 14.465) (end 33.75 23.5977) (width 0.25) (layer "F.Cu") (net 6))
 (segment (start 40.9769 26.5569) (end 39.75 25.33) (width 0.25) (layer "F.Cu") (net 6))
 (segment (start 35.7673 25.615) (end 36.225 25.615) (width 0.25) (layer "F.Cu") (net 6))
 (segment (start 40.9769 30.9918) (end 40.9769 26.5569) (width 0.25) (layer "F.Cu") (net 6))
 (segment (start 36.225 25.615) (end 39.465 25.615) (width 0.25) (layer "F.Cu") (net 6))
 (segment (start 40.2272 31.7415) (end 40.9769 30.9918) (width 0.25) (layer "F.Cu") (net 6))
 (segment (start 33.75 23.5977) (end 35.7673 25.615) (width 0.25) (layer "F.Cu") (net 6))
 (segment (start 20.9698 27.577) (end 27.7716 34.3788) (width 0.25) (layer "F.Cu") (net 4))
 (segment (start 31.275 24.345) (end 31.275 23.0676) (width 0.25) (layer "F.Cu") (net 4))
 (segment (start 20.1048 27.577) (end 20.9698 27.577) (width 0.25) (layer "F.Cu") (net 4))
 (segment (start 19.2866 26.7588) (end 20.1048 27.577) (width 0.25) (layer "F.Cu") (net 4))
 (via (at 31.275 23.0676) (size 0.6) (drill 0.3) (layers "F.Cu" "B.Cu") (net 4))
 (segment (start 27.7716 34.3788) (end 28.9483 33.2021) (width 0.25) (layer "B.Cu") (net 4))
 (segment (start 26.5806 29.7859) (end 26.5806 25.758) (width 0.25) (layer "B.Cu") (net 4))
 (segment (start 28.2679 30.6621) (end 27.4568 30.6621) (width 0.25) (layer "B.Cu") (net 4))
 (segment (start 26.5806 25.758) (end 29.271 23.0676) (width 0.25) (layer "B.Cu") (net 4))
 (segment (start 27.4568 30.6621) (end 26.5806 29.7859) (width 0.25) (layer "B.Cu") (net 4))
 (segment (start 28.9483 31.3425) (end 28.2679 30.6621) (width 0.25) (layer "B.Cu") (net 4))
 (segment (start 28.9483 33.2021) (end 28.9483 31.3425) (width 0.25) (layer "B.Cu") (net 4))
 (segment (start 29.271 23.0676) (end 31.275 23.0676) (width 0.25) (layer "B.Cu") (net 4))
 (segment (start 36.75 30.6832) (end 37.5301 29.9031) (width 0.25) (layer "F.Cu") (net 5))
 (segment (start 37.5301 27.8) (end 36.6151 26.885) (width 0.25) (layer "F.Cu") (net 5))
 (segment (start 36.75 30.6832) (end 36.75 34.115) (width 0.25) (layer "F.Cu") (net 5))
 (segment (start 44.645 28.5548) (end 44.645 30.6415) (width 0.25) (layer "F.Cu") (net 5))
 (segment (start 37.5301 29.9031) (end 37.5301 27.8) (width 0.25) (layer "F.Cu") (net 5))
 (segment (start 60.2531 35.4786) (end 49.4821 35.4786) (width 0.25) (layer "F.Cu") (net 5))
 (segment (start 44.645 26.25) (end 44.645 28.5548) (width 0.25) (layer "F.Cu") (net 5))
 (segment (start 49.4821 35.4786) (end 44.645 30.6415) (width 0.25) (layer "F.Cu") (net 5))
 (segment (start 36.6151 26.885) (end 36.225 26.885) (width 0.25) (layer "F.Cu") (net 5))
 (segment (start 66.615 29.1167) (end 60.2531 35.4786) (width 0.25) (layer "F.Cu") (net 5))
 (segment (start 66.615 26.25) (end 66.615 29.1167) (width 0.25) (layer "F.Cu") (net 5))
 (via (at 36.75 30.6832) (size 0.6) (drill 0.3) (layers "F.Cu" "B.Cu") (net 5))
 (via (at 44.645 30.6415) (size 0.6) (drill 0.3) (layers "F.Cu" "B.Cu") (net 5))
 (segment (start 36.7917 30.6415) (end 44.645 30.6415) (width 0.25) (layer "B.Cu") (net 5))
 (segment (start 36.75 30.6832) (end 36.7917 30.6415) (width 0.25) (layer "B.Cu") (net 5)))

